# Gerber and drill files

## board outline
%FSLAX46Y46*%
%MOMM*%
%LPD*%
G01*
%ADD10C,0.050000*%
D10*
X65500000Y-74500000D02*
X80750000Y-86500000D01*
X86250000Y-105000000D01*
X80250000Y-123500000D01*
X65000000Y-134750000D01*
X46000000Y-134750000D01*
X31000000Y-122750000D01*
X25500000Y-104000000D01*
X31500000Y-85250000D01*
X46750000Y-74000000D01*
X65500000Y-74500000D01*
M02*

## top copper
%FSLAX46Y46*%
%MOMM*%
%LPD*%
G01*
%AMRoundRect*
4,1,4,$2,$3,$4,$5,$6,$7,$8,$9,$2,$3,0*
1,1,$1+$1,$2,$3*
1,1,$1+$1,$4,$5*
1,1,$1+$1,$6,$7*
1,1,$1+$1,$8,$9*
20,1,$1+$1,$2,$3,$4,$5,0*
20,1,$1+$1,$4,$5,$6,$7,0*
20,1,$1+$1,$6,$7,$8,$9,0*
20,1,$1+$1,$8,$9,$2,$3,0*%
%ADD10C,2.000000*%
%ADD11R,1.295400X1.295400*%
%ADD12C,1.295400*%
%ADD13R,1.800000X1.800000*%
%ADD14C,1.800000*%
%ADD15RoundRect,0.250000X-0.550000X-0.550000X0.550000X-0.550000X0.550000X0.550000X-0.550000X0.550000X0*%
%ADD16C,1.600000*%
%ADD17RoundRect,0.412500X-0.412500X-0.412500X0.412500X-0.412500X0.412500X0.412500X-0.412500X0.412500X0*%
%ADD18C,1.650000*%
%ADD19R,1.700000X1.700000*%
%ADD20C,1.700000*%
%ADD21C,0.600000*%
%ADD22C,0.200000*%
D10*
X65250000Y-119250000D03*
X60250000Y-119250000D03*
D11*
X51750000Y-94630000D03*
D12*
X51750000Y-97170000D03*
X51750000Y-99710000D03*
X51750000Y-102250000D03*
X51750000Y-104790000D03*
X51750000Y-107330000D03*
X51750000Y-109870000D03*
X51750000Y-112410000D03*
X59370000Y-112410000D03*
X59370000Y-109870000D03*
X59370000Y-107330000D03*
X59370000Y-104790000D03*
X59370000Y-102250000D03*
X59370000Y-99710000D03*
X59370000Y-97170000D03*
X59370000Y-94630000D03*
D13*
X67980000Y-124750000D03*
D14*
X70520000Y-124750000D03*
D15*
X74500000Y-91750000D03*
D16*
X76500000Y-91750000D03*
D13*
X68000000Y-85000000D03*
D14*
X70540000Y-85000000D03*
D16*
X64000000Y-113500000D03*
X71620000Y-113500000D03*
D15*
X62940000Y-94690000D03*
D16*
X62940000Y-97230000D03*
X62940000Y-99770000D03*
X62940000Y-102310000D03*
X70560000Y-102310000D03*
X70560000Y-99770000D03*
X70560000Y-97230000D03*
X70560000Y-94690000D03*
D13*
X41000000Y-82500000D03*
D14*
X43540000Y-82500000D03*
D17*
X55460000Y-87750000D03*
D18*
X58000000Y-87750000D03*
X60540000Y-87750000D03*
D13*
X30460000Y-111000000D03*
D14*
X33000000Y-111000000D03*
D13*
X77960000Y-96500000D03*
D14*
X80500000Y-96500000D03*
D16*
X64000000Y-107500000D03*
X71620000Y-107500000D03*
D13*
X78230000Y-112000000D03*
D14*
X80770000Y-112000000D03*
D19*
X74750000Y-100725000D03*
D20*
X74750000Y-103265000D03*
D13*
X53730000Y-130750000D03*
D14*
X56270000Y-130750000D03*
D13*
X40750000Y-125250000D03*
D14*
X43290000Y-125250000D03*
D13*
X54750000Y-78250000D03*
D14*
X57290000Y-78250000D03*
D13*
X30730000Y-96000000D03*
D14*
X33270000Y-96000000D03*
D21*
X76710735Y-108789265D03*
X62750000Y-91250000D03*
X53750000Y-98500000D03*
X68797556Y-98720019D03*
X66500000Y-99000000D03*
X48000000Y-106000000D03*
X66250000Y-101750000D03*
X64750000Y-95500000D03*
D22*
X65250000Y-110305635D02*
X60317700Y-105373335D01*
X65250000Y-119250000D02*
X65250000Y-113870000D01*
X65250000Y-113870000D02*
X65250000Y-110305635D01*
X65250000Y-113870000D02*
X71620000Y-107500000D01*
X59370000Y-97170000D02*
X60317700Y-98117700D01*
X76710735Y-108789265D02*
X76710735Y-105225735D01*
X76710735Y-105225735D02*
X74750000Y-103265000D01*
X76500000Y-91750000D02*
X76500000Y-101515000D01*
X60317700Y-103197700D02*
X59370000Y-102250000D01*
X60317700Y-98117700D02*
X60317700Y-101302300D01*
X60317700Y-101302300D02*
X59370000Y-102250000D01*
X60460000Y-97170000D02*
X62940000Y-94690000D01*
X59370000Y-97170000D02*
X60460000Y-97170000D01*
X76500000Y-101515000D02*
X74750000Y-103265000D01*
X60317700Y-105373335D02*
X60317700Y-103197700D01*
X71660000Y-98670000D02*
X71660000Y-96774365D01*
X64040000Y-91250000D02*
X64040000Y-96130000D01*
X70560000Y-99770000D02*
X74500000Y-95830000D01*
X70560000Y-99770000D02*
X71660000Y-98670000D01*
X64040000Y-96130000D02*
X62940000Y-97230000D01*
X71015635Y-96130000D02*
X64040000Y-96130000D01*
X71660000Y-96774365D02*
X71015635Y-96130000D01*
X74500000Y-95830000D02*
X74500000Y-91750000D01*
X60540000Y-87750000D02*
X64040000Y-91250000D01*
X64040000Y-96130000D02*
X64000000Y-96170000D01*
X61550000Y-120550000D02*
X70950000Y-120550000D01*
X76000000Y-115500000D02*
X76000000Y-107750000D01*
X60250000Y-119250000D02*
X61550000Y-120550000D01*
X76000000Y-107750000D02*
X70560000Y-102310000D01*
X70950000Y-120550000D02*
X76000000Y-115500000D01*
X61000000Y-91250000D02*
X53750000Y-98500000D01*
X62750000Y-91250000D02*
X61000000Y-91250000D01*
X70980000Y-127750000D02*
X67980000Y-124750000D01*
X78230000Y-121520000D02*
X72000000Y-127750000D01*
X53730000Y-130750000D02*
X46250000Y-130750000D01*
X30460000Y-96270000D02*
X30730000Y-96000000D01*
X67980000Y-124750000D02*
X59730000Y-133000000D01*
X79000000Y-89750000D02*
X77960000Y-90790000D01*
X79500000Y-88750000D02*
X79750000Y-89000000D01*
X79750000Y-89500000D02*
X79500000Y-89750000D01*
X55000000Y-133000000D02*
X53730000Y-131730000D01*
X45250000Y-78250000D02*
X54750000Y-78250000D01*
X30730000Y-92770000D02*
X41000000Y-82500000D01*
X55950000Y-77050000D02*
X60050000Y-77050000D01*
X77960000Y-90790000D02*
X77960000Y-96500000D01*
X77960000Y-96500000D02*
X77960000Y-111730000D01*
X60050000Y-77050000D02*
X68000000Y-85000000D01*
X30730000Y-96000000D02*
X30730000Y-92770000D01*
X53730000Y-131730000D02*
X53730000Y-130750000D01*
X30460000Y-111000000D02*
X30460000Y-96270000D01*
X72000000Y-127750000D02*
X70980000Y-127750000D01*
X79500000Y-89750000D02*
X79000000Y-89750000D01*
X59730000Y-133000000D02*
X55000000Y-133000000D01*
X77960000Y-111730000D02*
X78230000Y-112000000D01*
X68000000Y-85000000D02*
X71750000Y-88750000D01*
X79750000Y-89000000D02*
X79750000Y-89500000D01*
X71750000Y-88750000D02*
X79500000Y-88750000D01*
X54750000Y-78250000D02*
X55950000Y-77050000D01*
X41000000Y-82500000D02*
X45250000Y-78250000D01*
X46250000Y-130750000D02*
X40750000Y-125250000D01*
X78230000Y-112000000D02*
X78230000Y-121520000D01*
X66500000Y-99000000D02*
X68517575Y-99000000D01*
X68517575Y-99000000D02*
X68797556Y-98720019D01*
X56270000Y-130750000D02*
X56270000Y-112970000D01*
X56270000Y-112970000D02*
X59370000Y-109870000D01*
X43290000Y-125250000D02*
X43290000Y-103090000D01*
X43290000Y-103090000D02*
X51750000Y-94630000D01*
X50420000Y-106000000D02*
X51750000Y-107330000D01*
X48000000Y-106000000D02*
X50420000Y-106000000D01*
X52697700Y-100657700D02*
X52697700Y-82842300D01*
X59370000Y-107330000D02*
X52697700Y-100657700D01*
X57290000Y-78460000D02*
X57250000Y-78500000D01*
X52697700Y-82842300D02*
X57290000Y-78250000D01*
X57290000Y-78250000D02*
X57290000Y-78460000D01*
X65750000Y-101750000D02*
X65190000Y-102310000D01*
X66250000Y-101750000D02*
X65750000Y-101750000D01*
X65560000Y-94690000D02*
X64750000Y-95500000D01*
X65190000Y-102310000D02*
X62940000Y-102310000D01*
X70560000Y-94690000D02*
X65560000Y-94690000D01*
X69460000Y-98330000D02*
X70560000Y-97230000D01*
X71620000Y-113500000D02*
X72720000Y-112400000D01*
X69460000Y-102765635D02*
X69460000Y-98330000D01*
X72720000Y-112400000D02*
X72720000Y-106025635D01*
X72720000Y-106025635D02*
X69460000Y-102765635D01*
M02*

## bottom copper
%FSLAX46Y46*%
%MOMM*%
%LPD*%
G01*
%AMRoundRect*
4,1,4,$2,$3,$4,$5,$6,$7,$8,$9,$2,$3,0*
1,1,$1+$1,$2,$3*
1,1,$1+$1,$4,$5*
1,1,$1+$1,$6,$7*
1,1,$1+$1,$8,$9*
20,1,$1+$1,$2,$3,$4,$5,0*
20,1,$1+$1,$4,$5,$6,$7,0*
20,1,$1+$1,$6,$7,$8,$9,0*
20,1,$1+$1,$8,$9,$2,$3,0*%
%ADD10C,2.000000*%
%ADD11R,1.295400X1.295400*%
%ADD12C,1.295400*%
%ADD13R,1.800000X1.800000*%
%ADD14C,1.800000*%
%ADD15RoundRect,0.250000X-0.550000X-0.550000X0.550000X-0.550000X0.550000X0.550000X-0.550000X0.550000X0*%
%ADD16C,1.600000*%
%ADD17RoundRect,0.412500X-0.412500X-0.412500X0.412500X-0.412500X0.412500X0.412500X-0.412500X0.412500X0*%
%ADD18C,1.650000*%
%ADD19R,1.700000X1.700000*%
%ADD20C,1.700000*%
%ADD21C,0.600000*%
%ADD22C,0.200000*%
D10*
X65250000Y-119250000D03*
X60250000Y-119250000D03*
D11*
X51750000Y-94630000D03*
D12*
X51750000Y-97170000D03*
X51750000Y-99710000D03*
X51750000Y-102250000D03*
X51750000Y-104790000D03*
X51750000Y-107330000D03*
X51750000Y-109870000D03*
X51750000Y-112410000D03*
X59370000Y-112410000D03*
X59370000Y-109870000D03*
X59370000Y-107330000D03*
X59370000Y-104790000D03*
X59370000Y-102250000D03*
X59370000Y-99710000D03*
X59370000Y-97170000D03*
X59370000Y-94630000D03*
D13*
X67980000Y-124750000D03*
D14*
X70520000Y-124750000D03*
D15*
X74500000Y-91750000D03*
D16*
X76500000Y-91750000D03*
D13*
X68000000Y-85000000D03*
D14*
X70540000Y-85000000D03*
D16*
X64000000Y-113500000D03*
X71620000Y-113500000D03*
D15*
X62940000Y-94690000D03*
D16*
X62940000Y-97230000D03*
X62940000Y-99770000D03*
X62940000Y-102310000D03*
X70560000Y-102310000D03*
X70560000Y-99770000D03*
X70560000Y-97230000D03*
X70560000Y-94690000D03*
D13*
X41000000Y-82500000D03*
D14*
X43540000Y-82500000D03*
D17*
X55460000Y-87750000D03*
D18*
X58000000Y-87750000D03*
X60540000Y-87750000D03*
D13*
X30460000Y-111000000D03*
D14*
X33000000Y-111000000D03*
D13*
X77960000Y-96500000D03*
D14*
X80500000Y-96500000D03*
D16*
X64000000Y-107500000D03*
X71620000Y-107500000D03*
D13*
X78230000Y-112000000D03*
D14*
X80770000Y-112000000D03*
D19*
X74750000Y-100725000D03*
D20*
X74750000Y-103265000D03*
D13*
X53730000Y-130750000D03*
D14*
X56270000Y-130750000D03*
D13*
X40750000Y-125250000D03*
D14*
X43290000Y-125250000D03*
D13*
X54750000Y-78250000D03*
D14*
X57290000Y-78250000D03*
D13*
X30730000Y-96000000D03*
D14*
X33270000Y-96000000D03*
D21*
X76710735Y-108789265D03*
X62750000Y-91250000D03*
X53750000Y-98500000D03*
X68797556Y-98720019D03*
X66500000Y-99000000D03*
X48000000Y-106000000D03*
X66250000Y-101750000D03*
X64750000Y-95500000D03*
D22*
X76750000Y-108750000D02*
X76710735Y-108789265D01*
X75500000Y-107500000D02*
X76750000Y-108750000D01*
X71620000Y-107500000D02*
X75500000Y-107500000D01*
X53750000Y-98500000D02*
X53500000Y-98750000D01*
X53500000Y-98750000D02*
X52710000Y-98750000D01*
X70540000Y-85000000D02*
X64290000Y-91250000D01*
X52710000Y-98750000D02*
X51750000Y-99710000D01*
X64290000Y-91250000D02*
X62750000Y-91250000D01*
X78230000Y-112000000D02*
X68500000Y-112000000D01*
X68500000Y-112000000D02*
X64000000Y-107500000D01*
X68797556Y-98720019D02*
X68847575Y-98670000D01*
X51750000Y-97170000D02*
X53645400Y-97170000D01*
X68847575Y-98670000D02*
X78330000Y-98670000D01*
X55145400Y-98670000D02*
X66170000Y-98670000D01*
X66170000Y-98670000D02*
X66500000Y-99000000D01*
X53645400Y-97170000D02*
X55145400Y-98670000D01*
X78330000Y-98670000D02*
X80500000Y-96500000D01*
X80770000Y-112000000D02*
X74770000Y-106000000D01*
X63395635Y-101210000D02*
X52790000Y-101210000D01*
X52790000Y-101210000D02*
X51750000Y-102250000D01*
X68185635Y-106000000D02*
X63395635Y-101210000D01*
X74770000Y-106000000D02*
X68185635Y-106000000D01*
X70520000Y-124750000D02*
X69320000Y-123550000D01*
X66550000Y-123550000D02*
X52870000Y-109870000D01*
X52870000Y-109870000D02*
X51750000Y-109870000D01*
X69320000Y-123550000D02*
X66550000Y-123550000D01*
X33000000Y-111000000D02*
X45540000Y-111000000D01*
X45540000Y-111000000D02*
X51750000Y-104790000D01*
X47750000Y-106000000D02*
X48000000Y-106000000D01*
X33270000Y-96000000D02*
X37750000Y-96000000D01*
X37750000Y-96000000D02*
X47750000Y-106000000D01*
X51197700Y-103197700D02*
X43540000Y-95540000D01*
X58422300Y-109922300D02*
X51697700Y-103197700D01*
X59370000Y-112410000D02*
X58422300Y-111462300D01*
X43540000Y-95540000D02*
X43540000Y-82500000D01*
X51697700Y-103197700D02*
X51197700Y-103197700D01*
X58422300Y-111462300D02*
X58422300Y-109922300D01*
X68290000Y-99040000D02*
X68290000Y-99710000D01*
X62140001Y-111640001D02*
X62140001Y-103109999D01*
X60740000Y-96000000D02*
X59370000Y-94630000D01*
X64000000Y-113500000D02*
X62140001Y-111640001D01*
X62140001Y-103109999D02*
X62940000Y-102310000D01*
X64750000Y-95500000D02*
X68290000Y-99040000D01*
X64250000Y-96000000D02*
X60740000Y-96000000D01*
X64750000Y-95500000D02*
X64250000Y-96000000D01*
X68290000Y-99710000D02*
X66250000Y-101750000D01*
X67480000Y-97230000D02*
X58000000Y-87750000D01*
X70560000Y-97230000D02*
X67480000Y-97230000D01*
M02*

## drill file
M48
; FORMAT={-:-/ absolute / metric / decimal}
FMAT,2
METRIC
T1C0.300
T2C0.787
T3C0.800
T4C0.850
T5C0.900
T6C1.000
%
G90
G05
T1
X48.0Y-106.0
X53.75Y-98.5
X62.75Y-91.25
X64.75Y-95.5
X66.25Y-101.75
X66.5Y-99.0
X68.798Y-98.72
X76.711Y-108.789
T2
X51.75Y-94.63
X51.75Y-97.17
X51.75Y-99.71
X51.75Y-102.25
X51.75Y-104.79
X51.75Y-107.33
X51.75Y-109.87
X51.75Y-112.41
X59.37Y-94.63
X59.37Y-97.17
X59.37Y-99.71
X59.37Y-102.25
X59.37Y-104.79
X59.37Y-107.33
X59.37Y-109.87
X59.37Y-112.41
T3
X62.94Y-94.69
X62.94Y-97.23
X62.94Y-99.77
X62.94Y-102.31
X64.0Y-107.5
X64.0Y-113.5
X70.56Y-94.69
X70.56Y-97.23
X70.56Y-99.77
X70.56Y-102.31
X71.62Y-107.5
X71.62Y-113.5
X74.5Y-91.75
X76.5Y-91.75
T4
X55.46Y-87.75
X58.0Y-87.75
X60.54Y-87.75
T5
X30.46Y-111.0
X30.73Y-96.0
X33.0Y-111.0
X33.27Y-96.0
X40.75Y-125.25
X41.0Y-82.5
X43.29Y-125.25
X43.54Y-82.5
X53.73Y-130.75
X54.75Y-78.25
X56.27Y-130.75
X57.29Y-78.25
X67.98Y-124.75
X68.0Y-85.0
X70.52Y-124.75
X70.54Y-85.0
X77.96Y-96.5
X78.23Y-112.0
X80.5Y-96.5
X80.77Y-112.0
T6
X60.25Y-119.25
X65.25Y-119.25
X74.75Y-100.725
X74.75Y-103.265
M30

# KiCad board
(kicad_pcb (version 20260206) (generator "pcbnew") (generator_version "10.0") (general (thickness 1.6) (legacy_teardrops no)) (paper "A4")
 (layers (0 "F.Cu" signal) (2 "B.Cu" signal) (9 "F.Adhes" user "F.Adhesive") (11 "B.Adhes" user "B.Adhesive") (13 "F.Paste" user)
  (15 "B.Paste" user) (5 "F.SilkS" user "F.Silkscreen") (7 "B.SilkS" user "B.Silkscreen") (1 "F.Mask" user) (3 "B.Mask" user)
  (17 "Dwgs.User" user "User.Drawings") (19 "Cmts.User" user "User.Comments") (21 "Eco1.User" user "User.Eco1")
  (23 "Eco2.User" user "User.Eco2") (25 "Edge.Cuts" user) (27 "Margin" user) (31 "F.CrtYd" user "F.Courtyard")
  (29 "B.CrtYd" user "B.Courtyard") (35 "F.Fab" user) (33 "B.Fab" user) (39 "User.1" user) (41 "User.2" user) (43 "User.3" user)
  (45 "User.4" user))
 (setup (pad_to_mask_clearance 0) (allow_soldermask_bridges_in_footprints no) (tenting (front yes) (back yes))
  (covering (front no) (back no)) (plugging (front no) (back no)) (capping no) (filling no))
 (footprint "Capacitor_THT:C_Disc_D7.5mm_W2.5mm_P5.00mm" (layer "F.Cu") (at 65.25 119.25 180)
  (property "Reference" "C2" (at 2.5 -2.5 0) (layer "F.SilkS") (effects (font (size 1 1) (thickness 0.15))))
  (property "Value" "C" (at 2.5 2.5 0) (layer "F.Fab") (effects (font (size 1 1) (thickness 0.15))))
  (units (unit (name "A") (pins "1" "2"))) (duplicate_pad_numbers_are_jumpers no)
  (pad "1" thru_hole circle (at 0 0 180) (size 2 2) (drill 1) (layers "*.Cu" "*.Mask") (remove_unused_layers no) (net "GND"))
  (pad "2" thru_hole circle (at 5 0 180) (size 2 2) (drill 1) (layers "*.Cu" "*.Mask") (remove_unused_layers no) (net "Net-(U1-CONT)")))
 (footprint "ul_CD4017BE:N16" (layer "F.Cu") (at 59.37 112.41)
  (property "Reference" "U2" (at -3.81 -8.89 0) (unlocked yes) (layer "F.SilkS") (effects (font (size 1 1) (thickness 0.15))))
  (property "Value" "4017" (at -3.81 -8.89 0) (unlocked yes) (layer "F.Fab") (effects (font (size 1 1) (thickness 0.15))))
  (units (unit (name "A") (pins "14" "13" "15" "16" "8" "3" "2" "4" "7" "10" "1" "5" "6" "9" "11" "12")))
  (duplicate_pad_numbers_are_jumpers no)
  (pad "1" thru_hole rect (at -7.62 -17.78) (size 1.2954 1.2954) (drill 0.7874) (layers "*.Cu" "*.Mask") (remove_unused_layers no)
   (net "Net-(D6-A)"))
  (pad "2" thru_hole circle (at -7.62 -15.24) (size 1.2954 1.2954) (drill 0.7874) (layers "*.Cu" "*.Mask") (remove_unused_layers no)
   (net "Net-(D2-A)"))
  (pad "3" thru_hole circle (at -7.62 -12.7) (size 1.2954 1.2954) (drill 0.7874) (layers "*.Cu" "*.Mask") (remove_unused_layers no)
   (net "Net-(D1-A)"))
  (pad "4" thru_hole circle (at -7.62 -10.16) (size 1.2954 1.2954) (drill 0.7874) (layers "*.Cu" "*.Mask") (remove_unused_layers no)
   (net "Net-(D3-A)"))
  (pad "5" thru_hole circle (at -7.62 -7.62) (size 1.2954 1.2954) (drill 0.7874) (layers "*.Cu" "*.Mask") (remove_unused_layers no)
   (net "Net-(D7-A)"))
  (pad "6" thru_hole circle (at -7.62 -5.08) (size 1.2954 1.2954) (drill 0.7874) (layers "*.Cu" "*.Mask") (remove_unused_layers no)
   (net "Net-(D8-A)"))
  (pad "7" thru_hole circle (at -7.62 -2.54) (size 1.2954 1.2954) (drill 0.7874) (layers "*.Cu" "*.Mask") (remove_unused_layers no)
   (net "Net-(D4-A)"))
  (pad "8" thru_hole circle (at -7.62 0) (size 1.2954 1.2954) (drill 0.7874) (layers "*.Cu" "*.Mask") (remove_unused_layers no)
   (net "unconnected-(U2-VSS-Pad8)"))
  (pad "9" thru_hole circle (at 0 0) (size 1.2954 1.2954) (drill 0.7874) (layers "*.Cu" "*.Mask") (remove_unused_layers no)
   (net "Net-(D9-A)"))
  (pad "10" thru_hole circle (at 0 -2.54) (size 1.2954 1.2954) (drill 0.7874) (layers "*.Cu" "*.Mask") (remove_unused_layers no)
   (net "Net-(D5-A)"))
  (pad "11" thru_hole circle (at 0 -5.08) (size 1.2954 1.2954) (drill 0.7874) (layers "*.Cu" "*.Mask") (remove_unused_layers no)
   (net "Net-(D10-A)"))
  (pad "12" thru_hole circle (at 0 -7.62) (size 1.2954 1.2954) (drill 0.7874) (layers "*.Cu" "*.Mask") (remove_unused_layers no)
   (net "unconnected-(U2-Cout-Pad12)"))
  (pad "13" thru_hole circle (at 0 -10.16) (size 1.2954 1.2954) (drill 0.7874) (layers "*.Cu" "*.Mask") (remove_unused_layers no)
   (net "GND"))
  (pad "14" thru_hole circle (at 0 -12.7) (size 1.2954 1.2954) (drill 0.7874) (layers "*.Cu" "*.Mask") (remove_unused_layers no)
   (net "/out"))
  (pad "15" thru_hole circle (at 0 -15.24) (size 1.2954 1.2954) (drill 0.7874) (layers "*.Cu" "*.Mask") (remove_unused_layers no)
   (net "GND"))
  (pad "16" thru_hole circle (at 0 -17.78) (size 1.2954 1.2954) (drill 0.7874) (layers "*.Cu" "*.Mask") (remove_unused_layers no)
   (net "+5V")))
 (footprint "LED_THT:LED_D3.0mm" (layer "F.Cu") (at 67.98 124.75)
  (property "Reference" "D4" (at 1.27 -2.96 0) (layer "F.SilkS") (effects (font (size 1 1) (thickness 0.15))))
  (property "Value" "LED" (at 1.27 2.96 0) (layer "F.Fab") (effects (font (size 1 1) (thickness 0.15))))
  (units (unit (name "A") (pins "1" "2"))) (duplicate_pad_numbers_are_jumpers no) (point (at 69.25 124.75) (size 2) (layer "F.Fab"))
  (pad "1" thru_hole rect (at 0 0) (size 1.8 1.8) (drill 0.9) (layers "*.Cu" "*.Mask") (remove_unused_layers no) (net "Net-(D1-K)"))
  (pad "2" thru_hole circle (at 2.54 0) (size 1.8 1.8) (drill 0.9) (layers "*.Cu" "*.Mask") (remove_unused_layers no) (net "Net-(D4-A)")))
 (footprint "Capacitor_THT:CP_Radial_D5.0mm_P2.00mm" (layer "F.Cu") (at 74.5 91.75)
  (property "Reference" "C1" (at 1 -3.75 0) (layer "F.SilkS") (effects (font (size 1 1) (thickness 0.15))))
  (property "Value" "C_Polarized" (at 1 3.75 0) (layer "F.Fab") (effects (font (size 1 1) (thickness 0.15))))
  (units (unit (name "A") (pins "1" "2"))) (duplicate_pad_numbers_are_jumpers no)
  (pad "1" thru_hole roundrect (at 0 0) (size 1.6 1.6) (drill 0.8) (layers "*.Cu" "*.Mask") (remove_unused_layers no)
   (roundrect_rratio 0.15625) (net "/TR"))
  (pad "2" thru_hole circle (at 2 0) (size 1.6 1.6) (drill 0.8) (layers "*.Cu" "*.Mask") (remove_unused_layers no) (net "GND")))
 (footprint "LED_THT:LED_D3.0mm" (layer "F.Cu") (at 68 85)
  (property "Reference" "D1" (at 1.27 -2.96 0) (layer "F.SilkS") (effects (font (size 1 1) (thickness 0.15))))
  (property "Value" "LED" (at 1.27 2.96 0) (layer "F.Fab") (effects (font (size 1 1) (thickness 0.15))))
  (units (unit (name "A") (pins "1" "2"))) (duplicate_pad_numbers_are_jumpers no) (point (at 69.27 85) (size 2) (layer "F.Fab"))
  (pad "1" thru_hole rect (at 0 0) (size 1.8 1.8) (drill 0.9) (layers "*.Cu" "*.Mask") (remove_unused_layers no) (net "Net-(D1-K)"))
  (pad "2" thru_hole circle (at 2.54 0) (size 1.8 1.8) (drill 0.9) (layers "*.Cu" "*.Mask") (remove_unused_layers no) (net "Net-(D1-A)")))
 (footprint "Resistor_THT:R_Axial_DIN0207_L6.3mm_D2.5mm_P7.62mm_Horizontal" (layer "F.Cu") (at 64 113.5)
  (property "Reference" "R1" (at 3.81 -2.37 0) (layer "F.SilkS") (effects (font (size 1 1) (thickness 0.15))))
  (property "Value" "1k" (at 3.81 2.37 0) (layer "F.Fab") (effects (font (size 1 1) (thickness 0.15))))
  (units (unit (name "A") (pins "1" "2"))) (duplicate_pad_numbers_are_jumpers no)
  (pad "1" thru_hole circle (at 0 0) (size 1.6 1.6) (drill 0.8) (layers "*.Cu" "*.Mask") (remove_unused_layers no) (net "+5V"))
  (pad "2" thru_hole circle (at 7.62 0) (size 1.6 1.6) (drill 0.8) (layers "*.Cu" "*.Mask") (remove_unused_layers no) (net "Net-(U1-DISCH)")))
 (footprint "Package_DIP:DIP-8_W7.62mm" (layer "F.Cu") (at 62.94 94.69)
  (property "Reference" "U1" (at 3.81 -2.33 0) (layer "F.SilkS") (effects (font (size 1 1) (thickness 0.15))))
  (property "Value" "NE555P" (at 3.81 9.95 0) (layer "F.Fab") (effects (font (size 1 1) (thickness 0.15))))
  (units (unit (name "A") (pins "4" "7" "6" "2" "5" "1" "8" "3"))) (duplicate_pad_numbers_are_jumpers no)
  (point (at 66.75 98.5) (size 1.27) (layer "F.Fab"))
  (pad "1" thru_hole roundrect (at 0 0) (size 1.6 1.6) (drill 0.8) (layers "*.Cu" "*.Mask") (remove_unused_layers no)
   (roundrect_rratio 0.15625) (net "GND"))
  (pad "2" thru_hole circle (at 0 2.54) (size 1.6 1.6) (drill 0.8) (layers "*.Cu" "*.Mask") (remove_unused_layers no) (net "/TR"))
  (pad "3" thru_hole circle (at 0 5.08) (size 1.6 1.6) (drill 0.8) (layers "*.Cu" "*.Mask") (remove_unused_layers no) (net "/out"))
  (pad "4" thru_hole circle (at 0 7.62) (size 1.6 1.6) (drill 0.8) (layers "*.Cu" "*.Mask") (remove_unused_layers no) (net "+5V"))
  (pad "5" thru_hole circle (at 7.62 7.62) (size 1.6 1.6) (drill 0.8) (layers "*.Cu" "*.Mask") (remove_unused_layers no)
   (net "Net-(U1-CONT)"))
  (pad "6" thru_hole circle (at 7.62 5.08) (size 1.6 1.6) (drill 0.8) (layers "*.Cu" "*.Mask") (remove_unused_layers no) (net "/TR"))
  (pad "7" thru_hole circle (at 7.62 2.54) (size 1.6 1.6) (drill 0.8) (layers "*.Cu" "*.Mask") (remove_unused_layers no)
   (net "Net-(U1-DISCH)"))
  (pad "8" thru_hole circle (at 7.62 0) (size 1.6 1.6) (drill 0.8) (layers "*.Cu" "*.Mask") (remove_unused_layers no) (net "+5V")))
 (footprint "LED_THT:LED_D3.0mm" (layer "F.Cu") (at 41 82.5)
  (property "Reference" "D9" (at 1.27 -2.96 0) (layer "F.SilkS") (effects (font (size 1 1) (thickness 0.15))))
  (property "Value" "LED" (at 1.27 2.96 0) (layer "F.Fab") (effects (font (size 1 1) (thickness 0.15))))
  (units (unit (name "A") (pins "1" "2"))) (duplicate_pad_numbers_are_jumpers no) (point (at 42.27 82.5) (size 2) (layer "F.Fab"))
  (pad "1" thru_hole rect (at 0 0) (size 1.8 1.8) (drill 0.9) (layers "*.Cu" "*.Mask") (remove_unused_layers no) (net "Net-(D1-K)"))
  (pad "2" thru_hole circle (at 2.54 0) (size 1.8 1.8) (drill 0.9) (layers "*.Cu" "*.Mask") (remove_unused_layers no) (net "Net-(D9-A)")))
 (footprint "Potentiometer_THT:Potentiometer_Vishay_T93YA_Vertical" (layer "F.Cu") (at 55.46 87.75)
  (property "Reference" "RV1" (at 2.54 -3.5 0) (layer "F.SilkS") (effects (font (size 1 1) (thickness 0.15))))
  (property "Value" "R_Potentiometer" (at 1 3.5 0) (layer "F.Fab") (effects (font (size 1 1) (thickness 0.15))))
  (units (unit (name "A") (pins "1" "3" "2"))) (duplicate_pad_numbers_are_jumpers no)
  (pad "1" thru_hole roundrect (at 0 0) (size 1.65 1.65) (drill 0.85) (layers "*.Cu" "*.Mask") (remove_unused_layers no)
   (roundrect_rratio 0.25) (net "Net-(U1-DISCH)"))
  (pad "2" thru_hole circle (at 2.54 0) (size 1.65 1.65) (drill 0.85) (layers "*.Cu" "*.Mask") (remove_unused_layers no)
   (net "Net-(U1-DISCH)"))
  (pad "3" thru_hole circle (at 5.08 0) (size 1.65 1.65) (drill 0.85) (layers "*.Cu" "*.Mask") (remove_unused_layers no) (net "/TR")))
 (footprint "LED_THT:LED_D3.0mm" (layer "F.Cu") (at 30.46 111)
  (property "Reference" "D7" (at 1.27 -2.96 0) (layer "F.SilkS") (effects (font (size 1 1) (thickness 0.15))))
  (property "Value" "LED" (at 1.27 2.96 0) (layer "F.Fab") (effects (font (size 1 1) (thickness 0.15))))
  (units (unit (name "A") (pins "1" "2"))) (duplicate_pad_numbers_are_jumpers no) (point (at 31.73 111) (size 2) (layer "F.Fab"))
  (pad "1" thru_hole rect (at 0 0) (size 1.8 1.8) (drill 0.9) (layers "*.Cu" "*.Mask") (remove_unused_layers no) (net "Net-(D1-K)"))
  (pad "2" thru_hole circle (at 2.54 0) (size 1.8 1.8) (drill 0.9) (layers "*.Cu" "*.Mask") (remove_unused_layers no) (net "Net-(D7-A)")))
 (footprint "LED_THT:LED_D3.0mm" (layer "F.Cu") (at 77.96 96.5)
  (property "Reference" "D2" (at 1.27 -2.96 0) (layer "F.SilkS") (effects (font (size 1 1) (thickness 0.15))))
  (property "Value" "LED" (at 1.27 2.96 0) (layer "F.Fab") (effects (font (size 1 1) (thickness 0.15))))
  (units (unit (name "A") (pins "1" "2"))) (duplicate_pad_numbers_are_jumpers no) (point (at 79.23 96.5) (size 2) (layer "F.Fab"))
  (pad "1" thru_hole rect (at 0 0) (size 1.8 1.8) (drill 0.9) (layers "*.Cu" "*.Mask") (remove_unused_layers no) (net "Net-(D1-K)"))
  (pad "2" thru_hole circle (at 2.54 0) (size 1.8 1.8) (drill 0.9) (layers "*.Cu" "*.Mask") (remove_unused_layers no) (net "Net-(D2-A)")))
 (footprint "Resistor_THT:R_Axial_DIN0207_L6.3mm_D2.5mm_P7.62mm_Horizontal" (layer "F.Cu") (at 64 107.5)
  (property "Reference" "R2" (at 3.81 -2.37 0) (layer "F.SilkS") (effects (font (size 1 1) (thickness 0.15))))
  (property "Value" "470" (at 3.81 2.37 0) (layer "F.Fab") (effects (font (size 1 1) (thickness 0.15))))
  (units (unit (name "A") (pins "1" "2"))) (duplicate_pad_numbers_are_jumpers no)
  (pad "1" thru_hole circle (at 0 0) (size 1.6 1.6) (drill 0.8) (layers "*.Cu" "*.Mask") (remove_unused_layers no) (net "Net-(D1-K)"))
  (pad "2" thru_hole circle (at 7.62 0) (size 1.6 1.6) (drill 0.8) (layers "*.Cu" "*.Mask") (remove_unused_layers no) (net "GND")))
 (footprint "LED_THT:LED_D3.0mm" (layer "F.Cu") (at 78.23 112)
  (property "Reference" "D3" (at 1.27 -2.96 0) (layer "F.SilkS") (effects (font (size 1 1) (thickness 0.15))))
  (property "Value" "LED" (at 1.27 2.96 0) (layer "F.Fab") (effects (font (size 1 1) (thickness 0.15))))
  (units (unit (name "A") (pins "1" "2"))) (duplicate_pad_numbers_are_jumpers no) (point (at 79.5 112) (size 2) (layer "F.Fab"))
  (pad "1" thru_hole rect (at 0 0) (size 1.8 1.8) (drill 0.9) (layers "*.Cu" "*.Mask") (remove_unused_layers no) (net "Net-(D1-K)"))
  (pad "2" thru_hole circle (at 2.54 0) (size 1.8 1.8) (drill 0.9) (layers "*.Cu" "*.Mask") (remove_unused_layers no) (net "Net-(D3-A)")))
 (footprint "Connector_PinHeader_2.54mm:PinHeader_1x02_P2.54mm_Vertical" (layer "F.Cu") (at 74.75 100.725)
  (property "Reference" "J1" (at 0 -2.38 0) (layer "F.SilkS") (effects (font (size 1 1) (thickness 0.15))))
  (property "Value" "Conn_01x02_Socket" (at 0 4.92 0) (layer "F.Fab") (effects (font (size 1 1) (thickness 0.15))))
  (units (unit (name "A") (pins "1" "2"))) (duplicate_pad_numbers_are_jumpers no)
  (pad "1" thru_hole rect (at 0 0) (size 1.7 1.7) (drill 1) (layers "*.Cu" "*.Mask") (remove_unused_layers no) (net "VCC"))
  (pad "2" thru_hole circle (at 0 2.54) (size 1.7 1.7) (drill 1) (layers "*.Cu" "*.Mask") (remove_unused_layers no) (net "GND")))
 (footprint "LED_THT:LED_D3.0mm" (layer "F.Cu") (at 53.73 130.75)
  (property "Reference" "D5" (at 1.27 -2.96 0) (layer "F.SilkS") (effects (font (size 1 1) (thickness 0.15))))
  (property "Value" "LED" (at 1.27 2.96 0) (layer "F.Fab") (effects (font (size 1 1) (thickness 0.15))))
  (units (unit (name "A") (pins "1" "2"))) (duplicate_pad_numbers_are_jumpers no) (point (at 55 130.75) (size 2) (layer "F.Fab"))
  (pad "1" thru_hole rect (at 0 0) (size 1.8 1.8) (drill 0.9) (layers "*.Cu" "*.Mask") (remove_unused_layers no) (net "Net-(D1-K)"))
  (pad "2" thru_hole circle (at 2.54 0) (size 1.8 1.8) (drill 0.9) (layers "*.Cu" "*.Mask") (remove_unused_layers no) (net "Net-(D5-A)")))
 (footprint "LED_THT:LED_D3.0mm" (layer "F.Cu") (at 40.75 125.25)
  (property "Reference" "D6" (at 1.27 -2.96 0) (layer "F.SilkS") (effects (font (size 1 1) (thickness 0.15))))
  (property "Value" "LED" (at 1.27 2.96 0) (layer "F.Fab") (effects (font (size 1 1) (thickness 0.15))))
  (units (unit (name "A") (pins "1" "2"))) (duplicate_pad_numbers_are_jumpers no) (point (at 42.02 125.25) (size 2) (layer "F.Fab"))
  (pad "1" thru_hole rect (at 0 0) (size 1.8 1.8) (drill 0.9) (layers "*.Cu" "*.Mask") (remove_unused_layers no) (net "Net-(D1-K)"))
  (pad "2" thru_hole circle (at 2.54 0) (size 1.8 1.8) (drill 0.9) (layers "*.Cu" "*.Mask") (remove_unused_layers no) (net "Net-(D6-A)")))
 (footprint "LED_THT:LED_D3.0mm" (layer "F.Cu") (at 54.75 78.25)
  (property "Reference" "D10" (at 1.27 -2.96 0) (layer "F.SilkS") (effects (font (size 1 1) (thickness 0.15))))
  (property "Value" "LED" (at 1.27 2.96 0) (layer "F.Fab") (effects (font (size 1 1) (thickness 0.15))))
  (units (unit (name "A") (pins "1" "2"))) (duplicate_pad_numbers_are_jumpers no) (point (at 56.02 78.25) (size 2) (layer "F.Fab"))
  (pad "1" thru_hole rect (at 0 0) (size 1.8 1.8) (drill 0.9) (layers "*.Cu" "*.Mask") (remove_unused_layers no) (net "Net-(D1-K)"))
  (pad "2" thru_hole circle (at 2.54 0) (size 1.8 1.8) (drill 0.9) (layers "*.Cu" "*.Mask") (remove_unused_layers no) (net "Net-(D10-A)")))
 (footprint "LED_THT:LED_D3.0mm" (layer "F.Cu") (at 30.73 96)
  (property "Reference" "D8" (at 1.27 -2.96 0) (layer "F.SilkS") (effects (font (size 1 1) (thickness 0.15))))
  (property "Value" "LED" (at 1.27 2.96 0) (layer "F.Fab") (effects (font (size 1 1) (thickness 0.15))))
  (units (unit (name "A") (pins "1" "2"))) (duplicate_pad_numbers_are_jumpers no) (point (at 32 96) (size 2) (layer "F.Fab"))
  (pad "1" thru_hole rect (at 0 0) (size 1.8 1.8) (drill 0.9) (layers "*.Cu" "*.Mask") (remove_unused_layers no) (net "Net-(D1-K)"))
  (pad "2" thru_hole circle (at 2.54 0) (size 1.8 1.8) (drill 0.9) (layers "*.Cu" "*.Mask") (remove_unused_layers no) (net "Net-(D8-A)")))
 (gr_poly
  (pts (xy 65.5 74.5) (xy 80.75 86.5) (xy 86.25 105) (xy 80.25 123.5) (xy 65 134.75) (xy 46 134.75) (xy 31 122.75) (xy 25.5 104)
   (xy 31.5 85.25) (xy 46.75 74))
  (stroke (width 0.05) (type solid)) (fill no) (layer "Edge.Cuts"))
 (segment (start 65.25 110.305635) (end 60.3177 105.373335) (width 0.2) (layer "F.Cu") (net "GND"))
 (segment (start 65.25 119.25) (end 65.25 113.87) (width 0.2) (layer "F.Cu") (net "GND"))
 (segment (start 65.25 113.87) (end 65.25 110.305635) (width 0.2) (layer "F.Cu") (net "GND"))
 (segment (start 65.25 113.87) (end 71.62 107.5) (width 0.2) (layer "F.Cu") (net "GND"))
 (segment (start 59.37 97.17) (end 60.3177 98.1177) (width 0.2) (layer "F.Cu") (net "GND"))
 (segment (start 76.710735 108.789265) (end 76.710735 105.225735) (width 0.2) (layer "F.Cu") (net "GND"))
 (segment (start 76.710735 105.225735) (end 74.75 103.265) (width 0.2) (layer "F.Cu") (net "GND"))
 (segment (start 76.5 91.75) (end 76.5 101.515) (width 0.2) (layer "F.Cu") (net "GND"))
 (segment (start 60.3177 103.1977) (end 59.37 102.25) (width 0.2) (layer "F.Cu") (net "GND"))
 (segment (start 60.3177 98.1177) (end 60.3177 101.3023) (width 0.2) (layer "F.Cu") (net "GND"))
 (segment (start 60.3177 101.3023) (end 59.37 102.25) (width 0.2) (layer "F.Cu") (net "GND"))
 (segment (start 60.46 97.17) (end 62.94 94.69) (width 0.2) (layer "F.Cu") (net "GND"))
 (segment (start 59.37 97.17) (end 60.46 97.17) (width 0.2) (layer "F.Cu") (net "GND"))
 (segment (start 76.5 101.515) (end 74.75 103.265) (width 0.2) (layer "F.Cu") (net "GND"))
 (segment (start 60.3177 105.373335) (end 60.3177 103.1977) (width 0.2) (layer "F.Cu") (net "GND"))
 (via (at 76.710735 108.789265) (size 0.6) (drill 0.3) (layers "F.Cu" "B.Cu") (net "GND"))
 (segment (start 76.75 108.75) (end 76.710735 108.789265) (width 0.2) (layer "B.Cu") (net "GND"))
 (segment (start 75.5 107.5) (end 76.75 108.75) (width 0.2) (layer "B.Cu") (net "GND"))
 (segment (start 71.62 107.5) (end 75.5 107.5) (width 0.2) (layer "B.Cu") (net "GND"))
 (segment (start 71.66 98.67) (end 71.66 96.774365) (width 0.2) (layer "F.Cu") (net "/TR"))
 (segment (start 64.04 91.25) (end 64.04 96.13) (width 0.2) (layer "F.Cu") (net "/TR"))
 (segment (start 70.56 99.77) (end 74.5 95.83) (width 0.2) (layer "F.Cu") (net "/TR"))
 (segment (start 70.56 99.77) (end 71.66 98.67) (width 0.2) (layer "F.Cu") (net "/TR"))
 (segment (start 64.04 96.13) (end 62.94 97.23) (width 0.2) (layer "F.Cu") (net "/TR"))
 (segment (start 71.015635 96.13) (end 64.04 96.13) (width 0.2) (layer "F.Cu") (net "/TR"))
 (segment (start 71.66 96.774365) (end 71.015635 96.13) (width 0.2) (layer "F.Cu") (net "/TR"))
 (segment (start 74.5 95.83) (end 74.5 91.75) (width 0.2) (layer "F.Cu") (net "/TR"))
 (segment (start 60.54 87.75) (end 64.04 91.25) (width 0.2) (layer "F.Cu") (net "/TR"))
 (segment (start 64.04 96.13) (end 64 96.17) (width 0.2) (layer "F.Cu") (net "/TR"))
 (segment (start 61.55 120.55) (end 70.95 120.55) (width 0.2) (layer "F.Cu") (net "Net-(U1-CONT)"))
 (segment (start 76 115.5) (end 76 107.75) (width 0.2) (layer "F.Cu") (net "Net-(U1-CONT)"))
 (segment (start 60.25 119.25) (end 61.55 120.55) (width 0.2) (layer "F.Cu") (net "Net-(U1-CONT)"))
 (segment (start 76 107.75) (end 70.56 102.31) (width 0.2) (layer "F.Cu") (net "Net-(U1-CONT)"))
 (segment (start 70.95 120.55) (end 76 115.5) (width 0.2) (layer "F.Cu") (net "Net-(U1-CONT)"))
 (segment (start 61 91.25) (end 53.75 98.5) (width 0.2) (layer "F.Cu") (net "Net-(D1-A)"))
 (segment (start 62.75 91.25) (end 61 91.25) (width 0.2) (layer "F.Cu") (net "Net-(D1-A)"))
 (via (at 62.75 91.25) (size 0.6) (drill 0.3) (layers "F.Cu" "B.Cu") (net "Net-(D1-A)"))
 (via (at 53.75 98.5) (size 0.6) (drill 0.3) (layers "F.Cu" "B.Cu") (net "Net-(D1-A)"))
 (segment (start 53.75 98.5) (end 53.5 98.75) (width 0.2) (layer "B.Cu") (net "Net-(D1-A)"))
 (segment (start 53.5 98.75) (end 52.71 98.75) (width 0.2) (layer "B.Cu") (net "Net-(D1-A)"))
 (segment (start 70.54 85) (end 64.29 91.25) (width 0.2) (layer "B.Cu") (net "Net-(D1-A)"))
 (segment (start 52.71 98.75) (end 51.75 99.71) (width 0.2) (layer "B.Cu") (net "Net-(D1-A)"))
 (segment (start 64.29 91.25) (end 62.75 91.25) (width 0.2) (layer "B.Cu") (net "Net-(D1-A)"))
 (segment (start 70.98 127.75) (end 67.98 124.75) (width 0.2) (layer "F.Cu") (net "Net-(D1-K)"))
 (segment (start 78.23 121.52) (end 72 127.75) (width 0.2) (layer "F.Cu") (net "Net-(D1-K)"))
 (segment (start 53.73 130.75) (end 46.25 130.75) (width 0.2) (layer "F.Cu") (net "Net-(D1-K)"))
 (segment (start 30.46 96.27) (end 30.73 96) (width 0.2) (layer "F.Cu") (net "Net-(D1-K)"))
 (segment (start 67.98 124.75) (end 59.73 133) (width 0.2) (layer "F.Cu") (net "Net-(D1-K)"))
 (segment (start 79 89.75) (end 77.96 90.79) (width 0.2) (layer "F.Cu") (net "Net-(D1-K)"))
 (segment (start 79.5 88.75) (end 79.75 89) (width 0.2) (layer "F.Cu") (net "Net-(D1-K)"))
 (segment (start 79.75 89.5) (end 79.5 89.75) (width 0.2) (layer "F.Cu") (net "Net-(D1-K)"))
 (segment (start 55 133) (end 53.73 131.73) (width 0.2) (layer "F.Cu") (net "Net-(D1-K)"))
 (segment (start 45.25 78.25) (end 54.75 78.25) (width 0.2) (layer "F.Cu") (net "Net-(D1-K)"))
 (segment (start 30.73 92.77) (end 41 82.5) (width 0.2) (layer "F.Cu") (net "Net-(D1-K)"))
 (segment (start 55.95 77.05) (end 60.05 77.05) (width 0.2) (layer "F.Cu") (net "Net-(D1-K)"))
 (segment (start 77.96 90.79) (end 77.96 96.5) (width 0.2) (layer "F.Cu") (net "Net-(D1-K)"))
 (segment (start 77.96 96.5) (end 77.96 111.73) (width 0.2) (layer "F.Cu") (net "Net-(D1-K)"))
 (segment (start 60.05 77.05) (end 68 85) (width 0.2) (layer "F.Cu") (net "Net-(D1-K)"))
 (segment (start 30.73 96) (end 30.73 92.77) (width 0.2) (layer "F.Cu") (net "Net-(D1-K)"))
 (segment (start 53.73 131.73) (end 53.73 130.75) (width 0.2) (layer "F.Cu") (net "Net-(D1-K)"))
 (segment (start 30.46 111) (end 30.46 96.27) (width 0.2) (layer "F.Cu") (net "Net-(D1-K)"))
 (segment (start 72 127.75) (end 70.98 127.75) (width 0.2) (layer "F.Cu") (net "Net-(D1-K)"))
 (segment (start 79.5 89.75) (end 79 89.75) (width 0.2) (layer "F.Cu") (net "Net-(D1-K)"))
 (segment (start 59.73 133) (end 55 133) (width 0.2) (layer "F.Cu") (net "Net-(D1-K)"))
 (segment (start 77.96 111.73) (end 78.23 112) (width 0.2) (layer "F.Cu") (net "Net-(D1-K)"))
 (segment (start 68 85) (end 71.75 88.75) (width 0.2) (layer "F.Cu") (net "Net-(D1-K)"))
 (segment (start 79.75 89) (end 79.75 89.5) (width 0.2) (layer "F.Cu") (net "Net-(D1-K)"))
 (segment (start 71.75 88.75) (end 79.5 88.75) (width 0.2) (layer "F.Cu") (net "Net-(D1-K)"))
 (segment (start 54.75 78.25) (end 55.95 77.05) (width 0.2) (layer "F.Cu") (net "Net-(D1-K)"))
 (segment (start 41 82.5) (end 45.25 78.25) (width 0.2) (layer "F.Cu") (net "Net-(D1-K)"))
 (segment (start 46.25 130.75) (end 40.75 125.25) (width 0.2) (layer "F.Cu") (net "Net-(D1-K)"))
 (segment (start 78.23 112) (end 78.23 121.52) (width 0.2) (layer "F.Cu") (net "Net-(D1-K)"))
 (segment (start 78.23 112) (end 68.5 112) (width 0.2) (layer "B.Cu") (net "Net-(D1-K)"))
 (segment (start 68.5 112) (end 64 107.5) (width 0.2) (layer "B.Cu") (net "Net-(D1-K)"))
 (segment (start 66.5 99) (end 68.517575 99) (width 0.2) (layer "F.Cu") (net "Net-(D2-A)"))
 (segment (start 68.517575 99) (end 68.797556 98.720019) (width 0.2) (layer "F.Cu") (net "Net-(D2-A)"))
 (via (at 68.797556 98.720019) (size 0.6) (drill 0.3) (layers "F.Cu" "B.Cu") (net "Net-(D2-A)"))
 (via (at 66.5 99) (size 0.6) (drill 0.3) (layers "F.Cu" "B.Cu") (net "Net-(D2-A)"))
 (segment (start 68.797556 98.720019) (end 68.847575 98.67) (width 0.2) (layer "B.Cu") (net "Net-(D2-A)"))
 (segment (start 51.75 97.17) (end 53.6454 97.17) (width 0.2) (layer "B.Cu") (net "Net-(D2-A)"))
 (segment (start 68.847575 98.67) (end 78.33 98.67) (width 0.2) (layer "B.Cu") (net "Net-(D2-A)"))
 (segment (start 55.1454 98.67) (end 66.17 98.67) (width 0.2) (layer "B.Cu") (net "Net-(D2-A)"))
 (segment (start 66.17 98.67) (end 66.5 99) (width 0.2) (layer "B.Cu") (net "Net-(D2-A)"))
 (segment (start 53.6454 97.17) (end 55.1454 98.67) (width 0.2) (layer "B.Cu") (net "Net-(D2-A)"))
 (segment (start 78.33 98.67) (end 80.5 96.5) (width 0.2) (layer "B.Cu") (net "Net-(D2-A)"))
 (segment (start 80.77 112) (end 74.77 106) (width 0.2) (layer "B.Cu") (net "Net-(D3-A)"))
 (segment (start 63.395635 101.21) (end 52.79 101.21) (width 0.2) (layer "B.Cu") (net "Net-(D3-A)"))
 (segment (start 52.79 101.21) (end 51.75 102.25) (width 0.2) (layer "B.Cu") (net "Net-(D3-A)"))
 (segment (start 68.185635 106) (end 63.395635 101.21) (width 0.2) (layer "B.Cu") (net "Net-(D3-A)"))
 (segment (start 74.77 106) (end 68.185635 106) (width 0.2) (layer "B.Cu") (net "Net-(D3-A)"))
 (segment (start 70.52 124.75) (end 69.32 123.55) (width 0.2) (layer "B.Cu") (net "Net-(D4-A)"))
 (segment (start 66.55 123.55) (end 52.87 109.87) (width 0.2) (layer "B.Cu") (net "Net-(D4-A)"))
 (segment (start 52.87 109.87) (end 51.75 109.87) (width 0.2) (layer "B.Cu") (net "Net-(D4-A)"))
 (segment (start 69.32 123.55) (end 66.55 123.55) (width 0.2) (layer "B.Cu") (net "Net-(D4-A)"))
 (segment (start 56.27 130.75) (end 56.27 112.97) (width 0.2) (layer "F.Cu") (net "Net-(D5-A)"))
 (segment (start 56.27 112.97) (end 59.37 109.87) (width 0.2) (layer "F.Cu") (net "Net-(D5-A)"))
 (segment (start 43.29 125.25) (end 43.29 103.09) (width 0.2) (layer "F.Cu") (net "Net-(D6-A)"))
 (segment (start 43.29 103.09) (end 51.75 94.63) (width 0.2) (layer "F.Cu") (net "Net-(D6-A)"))
 (segment (start 33 111) (end 45.54 111) (width 0.2) (layer "B.Cu") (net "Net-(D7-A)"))
 (segment (start 45.54 111) (end 51.75 104.79) (width 0.2) (layer "B.Cu") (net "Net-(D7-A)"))
 (segment (start 50.42 106) (end 51.75 107.33) (width 0.2) (layer "F.Cu") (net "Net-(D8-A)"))
 (segment (start 48 106) (end 50.42 106) (width 0.2) (layer "F.Cu") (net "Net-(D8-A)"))
 (via (at 48 106) (size 0.6) (drill 0.3) (layers "F.Cu" "B.Cu") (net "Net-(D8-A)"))
 (segment (start 47.75 106) (end 48 106) (width 0.2) (layer "B.Cu") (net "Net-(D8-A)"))
 (segment (start 33.27 96) (end 37.75 96) (width 0.2) (layer "B.Cu") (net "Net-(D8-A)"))
 (segment (start 37.75 96) (end 47.75 106) (width 0.2) (layer "B.Cu") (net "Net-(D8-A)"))
 (segment (start 51.1977 103.1977) (end 43.54 95.54) (width 0.2) (layer "B.Cu") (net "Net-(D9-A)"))
 (segment (start 58.4223 109.9223) (end 51.6977 103.1977) (width 0.2) (layer "B.Cu") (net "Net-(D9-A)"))
 (segment (start 59.37 112.41) (end 58.4223 111.4623) (width 0.2) (layer "B.Cu") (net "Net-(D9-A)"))
 (segment (start 43.54 95.54) (end 43.54 82.5) (width 0.2) (layer "B.Cu") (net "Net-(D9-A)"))
 (segment (start 51.6977 103.1977) (end 51.1977 103.1977) (width 0.2) (layer "B.Cu") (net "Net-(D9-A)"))
 (segment (start 58.4223 111.4623) (end 58.4223 109.9223) (width 0.2) (layer "B.Cu") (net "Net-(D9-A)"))
 (segment (start 52.6977 100.6577) (end 52.6977 82.8423) (width 0.2) (layer "F.Cu") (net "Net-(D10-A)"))
 (segment (start 59.37 107.33) (end 52.6977 100.6577) (width 0.2) (layer "F.Cu") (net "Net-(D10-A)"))
 (segment (start 57.29 78.46) (end 57.25 78.5) (width 0.2) (layer "F.Cu") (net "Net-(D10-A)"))
 (segment (start 52.6977 82.8423) (end 57.29 78.25) (width 0.2) (layer "F.Cu") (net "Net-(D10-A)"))
 (segment (start 57.29 78.25) (end 57.29 78.46) (width 0.2) (layer "F.Cu") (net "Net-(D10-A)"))
 (segment (start 65.75 101.75) (end 65.19 102.31) (width 0.2) (layer "F.Cu") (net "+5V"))
 (segment (start 66.25 101.75) (end 65.75 101.75) (width 0.2) (layer "F.Cu") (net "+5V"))
 (segment (start 65.56 94.69) (end 64.75 95.5) (width 0.2) (layer "F.Cu") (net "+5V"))
 (segment (start 65.19 102.31) (end 62.94 102.31) (width 0.2) (layer "F.Cu") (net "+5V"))
 (segment (start 70.56 94.69) (end 65.56 94.69) (width 0.2) (layer "F.Cu") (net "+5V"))
 (via (at 66.25 101.75) (size 0.6) (drill 0.3) (layers "F.Cu" "B.Cu") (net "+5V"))
 (via (at 64.75 95.5) (size 0.6) (drill 0.3) (layers "F.Cu" "B.Cu") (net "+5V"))
 (segment (start 68.29 99.04) (end 68.29 99.71) (width 0.2) (layer "B.Cu") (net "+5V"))
 (segment (start 62.140001 111.640001) (end 62.140001 103.109999) (width 0.2) (layer "B.Cu") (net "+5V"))
 (segment (start 60.74 96) (end 59.37 94.63) (width 0.2) (layer "B.Cu") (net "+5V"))
 (segment (start 64 113.5) (end 62.140001 111.640001) (width 0.2) (layer "B.Cu") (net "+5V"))
 (segment (start 62.140001 103.109999) (end 62.94 102.31) (width 0.2) (layer "B.Cu") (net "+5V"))
 (segment (start 64.75 95.5) (end 68.29 99.04) (width 0.2) (layer "B.Cu") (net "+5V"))
 (segment (start 64.25 96) (end 60.74 96) (width 0.2) (layer "B.Cu") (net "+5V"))
 (segment (start 64.75 95.5) (end 64.25 96) (width 0.2) (layer "B.Cu") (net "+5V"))
 (segment (start 68.29 99.71) (end 66.25 101.75) (width 0.2) (layer "B.Cu") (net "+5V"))
 (segment (start 69.46 98.33) (end 70.56 97.23) (width 0.2) (layer "F.Cu") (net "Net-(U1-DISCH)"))
 (segment (start 71.62 113.5) (end 72.72 112.4) (width 0.2) (layer "F.Cu") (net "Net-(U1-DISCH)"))
 (segment (start 69.46 102.765635) (end 69.46 98.33) (width 0.2) (layer "F.Cu") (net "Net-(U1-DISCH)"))
 (segment (start 72.72 112.4) (end 72.72 106.025635) (width 0.2) (layer "F.Cu") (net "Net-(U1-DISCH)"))
 (segment (start 72.72 106.025635) (end 69.46 102.765635) (width 0.2) (layer "F.Cu") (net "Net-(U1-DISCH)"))
 (segment (start 67.48 97.23) (end 58 87.75) (width 0.2) (layer "B.Cu") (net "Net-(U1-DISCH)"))
 (segment (start 70.56 97.23) (end 67.48 97.23) (width 0.2) (layer "B.Cu") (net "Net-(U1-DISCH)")))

